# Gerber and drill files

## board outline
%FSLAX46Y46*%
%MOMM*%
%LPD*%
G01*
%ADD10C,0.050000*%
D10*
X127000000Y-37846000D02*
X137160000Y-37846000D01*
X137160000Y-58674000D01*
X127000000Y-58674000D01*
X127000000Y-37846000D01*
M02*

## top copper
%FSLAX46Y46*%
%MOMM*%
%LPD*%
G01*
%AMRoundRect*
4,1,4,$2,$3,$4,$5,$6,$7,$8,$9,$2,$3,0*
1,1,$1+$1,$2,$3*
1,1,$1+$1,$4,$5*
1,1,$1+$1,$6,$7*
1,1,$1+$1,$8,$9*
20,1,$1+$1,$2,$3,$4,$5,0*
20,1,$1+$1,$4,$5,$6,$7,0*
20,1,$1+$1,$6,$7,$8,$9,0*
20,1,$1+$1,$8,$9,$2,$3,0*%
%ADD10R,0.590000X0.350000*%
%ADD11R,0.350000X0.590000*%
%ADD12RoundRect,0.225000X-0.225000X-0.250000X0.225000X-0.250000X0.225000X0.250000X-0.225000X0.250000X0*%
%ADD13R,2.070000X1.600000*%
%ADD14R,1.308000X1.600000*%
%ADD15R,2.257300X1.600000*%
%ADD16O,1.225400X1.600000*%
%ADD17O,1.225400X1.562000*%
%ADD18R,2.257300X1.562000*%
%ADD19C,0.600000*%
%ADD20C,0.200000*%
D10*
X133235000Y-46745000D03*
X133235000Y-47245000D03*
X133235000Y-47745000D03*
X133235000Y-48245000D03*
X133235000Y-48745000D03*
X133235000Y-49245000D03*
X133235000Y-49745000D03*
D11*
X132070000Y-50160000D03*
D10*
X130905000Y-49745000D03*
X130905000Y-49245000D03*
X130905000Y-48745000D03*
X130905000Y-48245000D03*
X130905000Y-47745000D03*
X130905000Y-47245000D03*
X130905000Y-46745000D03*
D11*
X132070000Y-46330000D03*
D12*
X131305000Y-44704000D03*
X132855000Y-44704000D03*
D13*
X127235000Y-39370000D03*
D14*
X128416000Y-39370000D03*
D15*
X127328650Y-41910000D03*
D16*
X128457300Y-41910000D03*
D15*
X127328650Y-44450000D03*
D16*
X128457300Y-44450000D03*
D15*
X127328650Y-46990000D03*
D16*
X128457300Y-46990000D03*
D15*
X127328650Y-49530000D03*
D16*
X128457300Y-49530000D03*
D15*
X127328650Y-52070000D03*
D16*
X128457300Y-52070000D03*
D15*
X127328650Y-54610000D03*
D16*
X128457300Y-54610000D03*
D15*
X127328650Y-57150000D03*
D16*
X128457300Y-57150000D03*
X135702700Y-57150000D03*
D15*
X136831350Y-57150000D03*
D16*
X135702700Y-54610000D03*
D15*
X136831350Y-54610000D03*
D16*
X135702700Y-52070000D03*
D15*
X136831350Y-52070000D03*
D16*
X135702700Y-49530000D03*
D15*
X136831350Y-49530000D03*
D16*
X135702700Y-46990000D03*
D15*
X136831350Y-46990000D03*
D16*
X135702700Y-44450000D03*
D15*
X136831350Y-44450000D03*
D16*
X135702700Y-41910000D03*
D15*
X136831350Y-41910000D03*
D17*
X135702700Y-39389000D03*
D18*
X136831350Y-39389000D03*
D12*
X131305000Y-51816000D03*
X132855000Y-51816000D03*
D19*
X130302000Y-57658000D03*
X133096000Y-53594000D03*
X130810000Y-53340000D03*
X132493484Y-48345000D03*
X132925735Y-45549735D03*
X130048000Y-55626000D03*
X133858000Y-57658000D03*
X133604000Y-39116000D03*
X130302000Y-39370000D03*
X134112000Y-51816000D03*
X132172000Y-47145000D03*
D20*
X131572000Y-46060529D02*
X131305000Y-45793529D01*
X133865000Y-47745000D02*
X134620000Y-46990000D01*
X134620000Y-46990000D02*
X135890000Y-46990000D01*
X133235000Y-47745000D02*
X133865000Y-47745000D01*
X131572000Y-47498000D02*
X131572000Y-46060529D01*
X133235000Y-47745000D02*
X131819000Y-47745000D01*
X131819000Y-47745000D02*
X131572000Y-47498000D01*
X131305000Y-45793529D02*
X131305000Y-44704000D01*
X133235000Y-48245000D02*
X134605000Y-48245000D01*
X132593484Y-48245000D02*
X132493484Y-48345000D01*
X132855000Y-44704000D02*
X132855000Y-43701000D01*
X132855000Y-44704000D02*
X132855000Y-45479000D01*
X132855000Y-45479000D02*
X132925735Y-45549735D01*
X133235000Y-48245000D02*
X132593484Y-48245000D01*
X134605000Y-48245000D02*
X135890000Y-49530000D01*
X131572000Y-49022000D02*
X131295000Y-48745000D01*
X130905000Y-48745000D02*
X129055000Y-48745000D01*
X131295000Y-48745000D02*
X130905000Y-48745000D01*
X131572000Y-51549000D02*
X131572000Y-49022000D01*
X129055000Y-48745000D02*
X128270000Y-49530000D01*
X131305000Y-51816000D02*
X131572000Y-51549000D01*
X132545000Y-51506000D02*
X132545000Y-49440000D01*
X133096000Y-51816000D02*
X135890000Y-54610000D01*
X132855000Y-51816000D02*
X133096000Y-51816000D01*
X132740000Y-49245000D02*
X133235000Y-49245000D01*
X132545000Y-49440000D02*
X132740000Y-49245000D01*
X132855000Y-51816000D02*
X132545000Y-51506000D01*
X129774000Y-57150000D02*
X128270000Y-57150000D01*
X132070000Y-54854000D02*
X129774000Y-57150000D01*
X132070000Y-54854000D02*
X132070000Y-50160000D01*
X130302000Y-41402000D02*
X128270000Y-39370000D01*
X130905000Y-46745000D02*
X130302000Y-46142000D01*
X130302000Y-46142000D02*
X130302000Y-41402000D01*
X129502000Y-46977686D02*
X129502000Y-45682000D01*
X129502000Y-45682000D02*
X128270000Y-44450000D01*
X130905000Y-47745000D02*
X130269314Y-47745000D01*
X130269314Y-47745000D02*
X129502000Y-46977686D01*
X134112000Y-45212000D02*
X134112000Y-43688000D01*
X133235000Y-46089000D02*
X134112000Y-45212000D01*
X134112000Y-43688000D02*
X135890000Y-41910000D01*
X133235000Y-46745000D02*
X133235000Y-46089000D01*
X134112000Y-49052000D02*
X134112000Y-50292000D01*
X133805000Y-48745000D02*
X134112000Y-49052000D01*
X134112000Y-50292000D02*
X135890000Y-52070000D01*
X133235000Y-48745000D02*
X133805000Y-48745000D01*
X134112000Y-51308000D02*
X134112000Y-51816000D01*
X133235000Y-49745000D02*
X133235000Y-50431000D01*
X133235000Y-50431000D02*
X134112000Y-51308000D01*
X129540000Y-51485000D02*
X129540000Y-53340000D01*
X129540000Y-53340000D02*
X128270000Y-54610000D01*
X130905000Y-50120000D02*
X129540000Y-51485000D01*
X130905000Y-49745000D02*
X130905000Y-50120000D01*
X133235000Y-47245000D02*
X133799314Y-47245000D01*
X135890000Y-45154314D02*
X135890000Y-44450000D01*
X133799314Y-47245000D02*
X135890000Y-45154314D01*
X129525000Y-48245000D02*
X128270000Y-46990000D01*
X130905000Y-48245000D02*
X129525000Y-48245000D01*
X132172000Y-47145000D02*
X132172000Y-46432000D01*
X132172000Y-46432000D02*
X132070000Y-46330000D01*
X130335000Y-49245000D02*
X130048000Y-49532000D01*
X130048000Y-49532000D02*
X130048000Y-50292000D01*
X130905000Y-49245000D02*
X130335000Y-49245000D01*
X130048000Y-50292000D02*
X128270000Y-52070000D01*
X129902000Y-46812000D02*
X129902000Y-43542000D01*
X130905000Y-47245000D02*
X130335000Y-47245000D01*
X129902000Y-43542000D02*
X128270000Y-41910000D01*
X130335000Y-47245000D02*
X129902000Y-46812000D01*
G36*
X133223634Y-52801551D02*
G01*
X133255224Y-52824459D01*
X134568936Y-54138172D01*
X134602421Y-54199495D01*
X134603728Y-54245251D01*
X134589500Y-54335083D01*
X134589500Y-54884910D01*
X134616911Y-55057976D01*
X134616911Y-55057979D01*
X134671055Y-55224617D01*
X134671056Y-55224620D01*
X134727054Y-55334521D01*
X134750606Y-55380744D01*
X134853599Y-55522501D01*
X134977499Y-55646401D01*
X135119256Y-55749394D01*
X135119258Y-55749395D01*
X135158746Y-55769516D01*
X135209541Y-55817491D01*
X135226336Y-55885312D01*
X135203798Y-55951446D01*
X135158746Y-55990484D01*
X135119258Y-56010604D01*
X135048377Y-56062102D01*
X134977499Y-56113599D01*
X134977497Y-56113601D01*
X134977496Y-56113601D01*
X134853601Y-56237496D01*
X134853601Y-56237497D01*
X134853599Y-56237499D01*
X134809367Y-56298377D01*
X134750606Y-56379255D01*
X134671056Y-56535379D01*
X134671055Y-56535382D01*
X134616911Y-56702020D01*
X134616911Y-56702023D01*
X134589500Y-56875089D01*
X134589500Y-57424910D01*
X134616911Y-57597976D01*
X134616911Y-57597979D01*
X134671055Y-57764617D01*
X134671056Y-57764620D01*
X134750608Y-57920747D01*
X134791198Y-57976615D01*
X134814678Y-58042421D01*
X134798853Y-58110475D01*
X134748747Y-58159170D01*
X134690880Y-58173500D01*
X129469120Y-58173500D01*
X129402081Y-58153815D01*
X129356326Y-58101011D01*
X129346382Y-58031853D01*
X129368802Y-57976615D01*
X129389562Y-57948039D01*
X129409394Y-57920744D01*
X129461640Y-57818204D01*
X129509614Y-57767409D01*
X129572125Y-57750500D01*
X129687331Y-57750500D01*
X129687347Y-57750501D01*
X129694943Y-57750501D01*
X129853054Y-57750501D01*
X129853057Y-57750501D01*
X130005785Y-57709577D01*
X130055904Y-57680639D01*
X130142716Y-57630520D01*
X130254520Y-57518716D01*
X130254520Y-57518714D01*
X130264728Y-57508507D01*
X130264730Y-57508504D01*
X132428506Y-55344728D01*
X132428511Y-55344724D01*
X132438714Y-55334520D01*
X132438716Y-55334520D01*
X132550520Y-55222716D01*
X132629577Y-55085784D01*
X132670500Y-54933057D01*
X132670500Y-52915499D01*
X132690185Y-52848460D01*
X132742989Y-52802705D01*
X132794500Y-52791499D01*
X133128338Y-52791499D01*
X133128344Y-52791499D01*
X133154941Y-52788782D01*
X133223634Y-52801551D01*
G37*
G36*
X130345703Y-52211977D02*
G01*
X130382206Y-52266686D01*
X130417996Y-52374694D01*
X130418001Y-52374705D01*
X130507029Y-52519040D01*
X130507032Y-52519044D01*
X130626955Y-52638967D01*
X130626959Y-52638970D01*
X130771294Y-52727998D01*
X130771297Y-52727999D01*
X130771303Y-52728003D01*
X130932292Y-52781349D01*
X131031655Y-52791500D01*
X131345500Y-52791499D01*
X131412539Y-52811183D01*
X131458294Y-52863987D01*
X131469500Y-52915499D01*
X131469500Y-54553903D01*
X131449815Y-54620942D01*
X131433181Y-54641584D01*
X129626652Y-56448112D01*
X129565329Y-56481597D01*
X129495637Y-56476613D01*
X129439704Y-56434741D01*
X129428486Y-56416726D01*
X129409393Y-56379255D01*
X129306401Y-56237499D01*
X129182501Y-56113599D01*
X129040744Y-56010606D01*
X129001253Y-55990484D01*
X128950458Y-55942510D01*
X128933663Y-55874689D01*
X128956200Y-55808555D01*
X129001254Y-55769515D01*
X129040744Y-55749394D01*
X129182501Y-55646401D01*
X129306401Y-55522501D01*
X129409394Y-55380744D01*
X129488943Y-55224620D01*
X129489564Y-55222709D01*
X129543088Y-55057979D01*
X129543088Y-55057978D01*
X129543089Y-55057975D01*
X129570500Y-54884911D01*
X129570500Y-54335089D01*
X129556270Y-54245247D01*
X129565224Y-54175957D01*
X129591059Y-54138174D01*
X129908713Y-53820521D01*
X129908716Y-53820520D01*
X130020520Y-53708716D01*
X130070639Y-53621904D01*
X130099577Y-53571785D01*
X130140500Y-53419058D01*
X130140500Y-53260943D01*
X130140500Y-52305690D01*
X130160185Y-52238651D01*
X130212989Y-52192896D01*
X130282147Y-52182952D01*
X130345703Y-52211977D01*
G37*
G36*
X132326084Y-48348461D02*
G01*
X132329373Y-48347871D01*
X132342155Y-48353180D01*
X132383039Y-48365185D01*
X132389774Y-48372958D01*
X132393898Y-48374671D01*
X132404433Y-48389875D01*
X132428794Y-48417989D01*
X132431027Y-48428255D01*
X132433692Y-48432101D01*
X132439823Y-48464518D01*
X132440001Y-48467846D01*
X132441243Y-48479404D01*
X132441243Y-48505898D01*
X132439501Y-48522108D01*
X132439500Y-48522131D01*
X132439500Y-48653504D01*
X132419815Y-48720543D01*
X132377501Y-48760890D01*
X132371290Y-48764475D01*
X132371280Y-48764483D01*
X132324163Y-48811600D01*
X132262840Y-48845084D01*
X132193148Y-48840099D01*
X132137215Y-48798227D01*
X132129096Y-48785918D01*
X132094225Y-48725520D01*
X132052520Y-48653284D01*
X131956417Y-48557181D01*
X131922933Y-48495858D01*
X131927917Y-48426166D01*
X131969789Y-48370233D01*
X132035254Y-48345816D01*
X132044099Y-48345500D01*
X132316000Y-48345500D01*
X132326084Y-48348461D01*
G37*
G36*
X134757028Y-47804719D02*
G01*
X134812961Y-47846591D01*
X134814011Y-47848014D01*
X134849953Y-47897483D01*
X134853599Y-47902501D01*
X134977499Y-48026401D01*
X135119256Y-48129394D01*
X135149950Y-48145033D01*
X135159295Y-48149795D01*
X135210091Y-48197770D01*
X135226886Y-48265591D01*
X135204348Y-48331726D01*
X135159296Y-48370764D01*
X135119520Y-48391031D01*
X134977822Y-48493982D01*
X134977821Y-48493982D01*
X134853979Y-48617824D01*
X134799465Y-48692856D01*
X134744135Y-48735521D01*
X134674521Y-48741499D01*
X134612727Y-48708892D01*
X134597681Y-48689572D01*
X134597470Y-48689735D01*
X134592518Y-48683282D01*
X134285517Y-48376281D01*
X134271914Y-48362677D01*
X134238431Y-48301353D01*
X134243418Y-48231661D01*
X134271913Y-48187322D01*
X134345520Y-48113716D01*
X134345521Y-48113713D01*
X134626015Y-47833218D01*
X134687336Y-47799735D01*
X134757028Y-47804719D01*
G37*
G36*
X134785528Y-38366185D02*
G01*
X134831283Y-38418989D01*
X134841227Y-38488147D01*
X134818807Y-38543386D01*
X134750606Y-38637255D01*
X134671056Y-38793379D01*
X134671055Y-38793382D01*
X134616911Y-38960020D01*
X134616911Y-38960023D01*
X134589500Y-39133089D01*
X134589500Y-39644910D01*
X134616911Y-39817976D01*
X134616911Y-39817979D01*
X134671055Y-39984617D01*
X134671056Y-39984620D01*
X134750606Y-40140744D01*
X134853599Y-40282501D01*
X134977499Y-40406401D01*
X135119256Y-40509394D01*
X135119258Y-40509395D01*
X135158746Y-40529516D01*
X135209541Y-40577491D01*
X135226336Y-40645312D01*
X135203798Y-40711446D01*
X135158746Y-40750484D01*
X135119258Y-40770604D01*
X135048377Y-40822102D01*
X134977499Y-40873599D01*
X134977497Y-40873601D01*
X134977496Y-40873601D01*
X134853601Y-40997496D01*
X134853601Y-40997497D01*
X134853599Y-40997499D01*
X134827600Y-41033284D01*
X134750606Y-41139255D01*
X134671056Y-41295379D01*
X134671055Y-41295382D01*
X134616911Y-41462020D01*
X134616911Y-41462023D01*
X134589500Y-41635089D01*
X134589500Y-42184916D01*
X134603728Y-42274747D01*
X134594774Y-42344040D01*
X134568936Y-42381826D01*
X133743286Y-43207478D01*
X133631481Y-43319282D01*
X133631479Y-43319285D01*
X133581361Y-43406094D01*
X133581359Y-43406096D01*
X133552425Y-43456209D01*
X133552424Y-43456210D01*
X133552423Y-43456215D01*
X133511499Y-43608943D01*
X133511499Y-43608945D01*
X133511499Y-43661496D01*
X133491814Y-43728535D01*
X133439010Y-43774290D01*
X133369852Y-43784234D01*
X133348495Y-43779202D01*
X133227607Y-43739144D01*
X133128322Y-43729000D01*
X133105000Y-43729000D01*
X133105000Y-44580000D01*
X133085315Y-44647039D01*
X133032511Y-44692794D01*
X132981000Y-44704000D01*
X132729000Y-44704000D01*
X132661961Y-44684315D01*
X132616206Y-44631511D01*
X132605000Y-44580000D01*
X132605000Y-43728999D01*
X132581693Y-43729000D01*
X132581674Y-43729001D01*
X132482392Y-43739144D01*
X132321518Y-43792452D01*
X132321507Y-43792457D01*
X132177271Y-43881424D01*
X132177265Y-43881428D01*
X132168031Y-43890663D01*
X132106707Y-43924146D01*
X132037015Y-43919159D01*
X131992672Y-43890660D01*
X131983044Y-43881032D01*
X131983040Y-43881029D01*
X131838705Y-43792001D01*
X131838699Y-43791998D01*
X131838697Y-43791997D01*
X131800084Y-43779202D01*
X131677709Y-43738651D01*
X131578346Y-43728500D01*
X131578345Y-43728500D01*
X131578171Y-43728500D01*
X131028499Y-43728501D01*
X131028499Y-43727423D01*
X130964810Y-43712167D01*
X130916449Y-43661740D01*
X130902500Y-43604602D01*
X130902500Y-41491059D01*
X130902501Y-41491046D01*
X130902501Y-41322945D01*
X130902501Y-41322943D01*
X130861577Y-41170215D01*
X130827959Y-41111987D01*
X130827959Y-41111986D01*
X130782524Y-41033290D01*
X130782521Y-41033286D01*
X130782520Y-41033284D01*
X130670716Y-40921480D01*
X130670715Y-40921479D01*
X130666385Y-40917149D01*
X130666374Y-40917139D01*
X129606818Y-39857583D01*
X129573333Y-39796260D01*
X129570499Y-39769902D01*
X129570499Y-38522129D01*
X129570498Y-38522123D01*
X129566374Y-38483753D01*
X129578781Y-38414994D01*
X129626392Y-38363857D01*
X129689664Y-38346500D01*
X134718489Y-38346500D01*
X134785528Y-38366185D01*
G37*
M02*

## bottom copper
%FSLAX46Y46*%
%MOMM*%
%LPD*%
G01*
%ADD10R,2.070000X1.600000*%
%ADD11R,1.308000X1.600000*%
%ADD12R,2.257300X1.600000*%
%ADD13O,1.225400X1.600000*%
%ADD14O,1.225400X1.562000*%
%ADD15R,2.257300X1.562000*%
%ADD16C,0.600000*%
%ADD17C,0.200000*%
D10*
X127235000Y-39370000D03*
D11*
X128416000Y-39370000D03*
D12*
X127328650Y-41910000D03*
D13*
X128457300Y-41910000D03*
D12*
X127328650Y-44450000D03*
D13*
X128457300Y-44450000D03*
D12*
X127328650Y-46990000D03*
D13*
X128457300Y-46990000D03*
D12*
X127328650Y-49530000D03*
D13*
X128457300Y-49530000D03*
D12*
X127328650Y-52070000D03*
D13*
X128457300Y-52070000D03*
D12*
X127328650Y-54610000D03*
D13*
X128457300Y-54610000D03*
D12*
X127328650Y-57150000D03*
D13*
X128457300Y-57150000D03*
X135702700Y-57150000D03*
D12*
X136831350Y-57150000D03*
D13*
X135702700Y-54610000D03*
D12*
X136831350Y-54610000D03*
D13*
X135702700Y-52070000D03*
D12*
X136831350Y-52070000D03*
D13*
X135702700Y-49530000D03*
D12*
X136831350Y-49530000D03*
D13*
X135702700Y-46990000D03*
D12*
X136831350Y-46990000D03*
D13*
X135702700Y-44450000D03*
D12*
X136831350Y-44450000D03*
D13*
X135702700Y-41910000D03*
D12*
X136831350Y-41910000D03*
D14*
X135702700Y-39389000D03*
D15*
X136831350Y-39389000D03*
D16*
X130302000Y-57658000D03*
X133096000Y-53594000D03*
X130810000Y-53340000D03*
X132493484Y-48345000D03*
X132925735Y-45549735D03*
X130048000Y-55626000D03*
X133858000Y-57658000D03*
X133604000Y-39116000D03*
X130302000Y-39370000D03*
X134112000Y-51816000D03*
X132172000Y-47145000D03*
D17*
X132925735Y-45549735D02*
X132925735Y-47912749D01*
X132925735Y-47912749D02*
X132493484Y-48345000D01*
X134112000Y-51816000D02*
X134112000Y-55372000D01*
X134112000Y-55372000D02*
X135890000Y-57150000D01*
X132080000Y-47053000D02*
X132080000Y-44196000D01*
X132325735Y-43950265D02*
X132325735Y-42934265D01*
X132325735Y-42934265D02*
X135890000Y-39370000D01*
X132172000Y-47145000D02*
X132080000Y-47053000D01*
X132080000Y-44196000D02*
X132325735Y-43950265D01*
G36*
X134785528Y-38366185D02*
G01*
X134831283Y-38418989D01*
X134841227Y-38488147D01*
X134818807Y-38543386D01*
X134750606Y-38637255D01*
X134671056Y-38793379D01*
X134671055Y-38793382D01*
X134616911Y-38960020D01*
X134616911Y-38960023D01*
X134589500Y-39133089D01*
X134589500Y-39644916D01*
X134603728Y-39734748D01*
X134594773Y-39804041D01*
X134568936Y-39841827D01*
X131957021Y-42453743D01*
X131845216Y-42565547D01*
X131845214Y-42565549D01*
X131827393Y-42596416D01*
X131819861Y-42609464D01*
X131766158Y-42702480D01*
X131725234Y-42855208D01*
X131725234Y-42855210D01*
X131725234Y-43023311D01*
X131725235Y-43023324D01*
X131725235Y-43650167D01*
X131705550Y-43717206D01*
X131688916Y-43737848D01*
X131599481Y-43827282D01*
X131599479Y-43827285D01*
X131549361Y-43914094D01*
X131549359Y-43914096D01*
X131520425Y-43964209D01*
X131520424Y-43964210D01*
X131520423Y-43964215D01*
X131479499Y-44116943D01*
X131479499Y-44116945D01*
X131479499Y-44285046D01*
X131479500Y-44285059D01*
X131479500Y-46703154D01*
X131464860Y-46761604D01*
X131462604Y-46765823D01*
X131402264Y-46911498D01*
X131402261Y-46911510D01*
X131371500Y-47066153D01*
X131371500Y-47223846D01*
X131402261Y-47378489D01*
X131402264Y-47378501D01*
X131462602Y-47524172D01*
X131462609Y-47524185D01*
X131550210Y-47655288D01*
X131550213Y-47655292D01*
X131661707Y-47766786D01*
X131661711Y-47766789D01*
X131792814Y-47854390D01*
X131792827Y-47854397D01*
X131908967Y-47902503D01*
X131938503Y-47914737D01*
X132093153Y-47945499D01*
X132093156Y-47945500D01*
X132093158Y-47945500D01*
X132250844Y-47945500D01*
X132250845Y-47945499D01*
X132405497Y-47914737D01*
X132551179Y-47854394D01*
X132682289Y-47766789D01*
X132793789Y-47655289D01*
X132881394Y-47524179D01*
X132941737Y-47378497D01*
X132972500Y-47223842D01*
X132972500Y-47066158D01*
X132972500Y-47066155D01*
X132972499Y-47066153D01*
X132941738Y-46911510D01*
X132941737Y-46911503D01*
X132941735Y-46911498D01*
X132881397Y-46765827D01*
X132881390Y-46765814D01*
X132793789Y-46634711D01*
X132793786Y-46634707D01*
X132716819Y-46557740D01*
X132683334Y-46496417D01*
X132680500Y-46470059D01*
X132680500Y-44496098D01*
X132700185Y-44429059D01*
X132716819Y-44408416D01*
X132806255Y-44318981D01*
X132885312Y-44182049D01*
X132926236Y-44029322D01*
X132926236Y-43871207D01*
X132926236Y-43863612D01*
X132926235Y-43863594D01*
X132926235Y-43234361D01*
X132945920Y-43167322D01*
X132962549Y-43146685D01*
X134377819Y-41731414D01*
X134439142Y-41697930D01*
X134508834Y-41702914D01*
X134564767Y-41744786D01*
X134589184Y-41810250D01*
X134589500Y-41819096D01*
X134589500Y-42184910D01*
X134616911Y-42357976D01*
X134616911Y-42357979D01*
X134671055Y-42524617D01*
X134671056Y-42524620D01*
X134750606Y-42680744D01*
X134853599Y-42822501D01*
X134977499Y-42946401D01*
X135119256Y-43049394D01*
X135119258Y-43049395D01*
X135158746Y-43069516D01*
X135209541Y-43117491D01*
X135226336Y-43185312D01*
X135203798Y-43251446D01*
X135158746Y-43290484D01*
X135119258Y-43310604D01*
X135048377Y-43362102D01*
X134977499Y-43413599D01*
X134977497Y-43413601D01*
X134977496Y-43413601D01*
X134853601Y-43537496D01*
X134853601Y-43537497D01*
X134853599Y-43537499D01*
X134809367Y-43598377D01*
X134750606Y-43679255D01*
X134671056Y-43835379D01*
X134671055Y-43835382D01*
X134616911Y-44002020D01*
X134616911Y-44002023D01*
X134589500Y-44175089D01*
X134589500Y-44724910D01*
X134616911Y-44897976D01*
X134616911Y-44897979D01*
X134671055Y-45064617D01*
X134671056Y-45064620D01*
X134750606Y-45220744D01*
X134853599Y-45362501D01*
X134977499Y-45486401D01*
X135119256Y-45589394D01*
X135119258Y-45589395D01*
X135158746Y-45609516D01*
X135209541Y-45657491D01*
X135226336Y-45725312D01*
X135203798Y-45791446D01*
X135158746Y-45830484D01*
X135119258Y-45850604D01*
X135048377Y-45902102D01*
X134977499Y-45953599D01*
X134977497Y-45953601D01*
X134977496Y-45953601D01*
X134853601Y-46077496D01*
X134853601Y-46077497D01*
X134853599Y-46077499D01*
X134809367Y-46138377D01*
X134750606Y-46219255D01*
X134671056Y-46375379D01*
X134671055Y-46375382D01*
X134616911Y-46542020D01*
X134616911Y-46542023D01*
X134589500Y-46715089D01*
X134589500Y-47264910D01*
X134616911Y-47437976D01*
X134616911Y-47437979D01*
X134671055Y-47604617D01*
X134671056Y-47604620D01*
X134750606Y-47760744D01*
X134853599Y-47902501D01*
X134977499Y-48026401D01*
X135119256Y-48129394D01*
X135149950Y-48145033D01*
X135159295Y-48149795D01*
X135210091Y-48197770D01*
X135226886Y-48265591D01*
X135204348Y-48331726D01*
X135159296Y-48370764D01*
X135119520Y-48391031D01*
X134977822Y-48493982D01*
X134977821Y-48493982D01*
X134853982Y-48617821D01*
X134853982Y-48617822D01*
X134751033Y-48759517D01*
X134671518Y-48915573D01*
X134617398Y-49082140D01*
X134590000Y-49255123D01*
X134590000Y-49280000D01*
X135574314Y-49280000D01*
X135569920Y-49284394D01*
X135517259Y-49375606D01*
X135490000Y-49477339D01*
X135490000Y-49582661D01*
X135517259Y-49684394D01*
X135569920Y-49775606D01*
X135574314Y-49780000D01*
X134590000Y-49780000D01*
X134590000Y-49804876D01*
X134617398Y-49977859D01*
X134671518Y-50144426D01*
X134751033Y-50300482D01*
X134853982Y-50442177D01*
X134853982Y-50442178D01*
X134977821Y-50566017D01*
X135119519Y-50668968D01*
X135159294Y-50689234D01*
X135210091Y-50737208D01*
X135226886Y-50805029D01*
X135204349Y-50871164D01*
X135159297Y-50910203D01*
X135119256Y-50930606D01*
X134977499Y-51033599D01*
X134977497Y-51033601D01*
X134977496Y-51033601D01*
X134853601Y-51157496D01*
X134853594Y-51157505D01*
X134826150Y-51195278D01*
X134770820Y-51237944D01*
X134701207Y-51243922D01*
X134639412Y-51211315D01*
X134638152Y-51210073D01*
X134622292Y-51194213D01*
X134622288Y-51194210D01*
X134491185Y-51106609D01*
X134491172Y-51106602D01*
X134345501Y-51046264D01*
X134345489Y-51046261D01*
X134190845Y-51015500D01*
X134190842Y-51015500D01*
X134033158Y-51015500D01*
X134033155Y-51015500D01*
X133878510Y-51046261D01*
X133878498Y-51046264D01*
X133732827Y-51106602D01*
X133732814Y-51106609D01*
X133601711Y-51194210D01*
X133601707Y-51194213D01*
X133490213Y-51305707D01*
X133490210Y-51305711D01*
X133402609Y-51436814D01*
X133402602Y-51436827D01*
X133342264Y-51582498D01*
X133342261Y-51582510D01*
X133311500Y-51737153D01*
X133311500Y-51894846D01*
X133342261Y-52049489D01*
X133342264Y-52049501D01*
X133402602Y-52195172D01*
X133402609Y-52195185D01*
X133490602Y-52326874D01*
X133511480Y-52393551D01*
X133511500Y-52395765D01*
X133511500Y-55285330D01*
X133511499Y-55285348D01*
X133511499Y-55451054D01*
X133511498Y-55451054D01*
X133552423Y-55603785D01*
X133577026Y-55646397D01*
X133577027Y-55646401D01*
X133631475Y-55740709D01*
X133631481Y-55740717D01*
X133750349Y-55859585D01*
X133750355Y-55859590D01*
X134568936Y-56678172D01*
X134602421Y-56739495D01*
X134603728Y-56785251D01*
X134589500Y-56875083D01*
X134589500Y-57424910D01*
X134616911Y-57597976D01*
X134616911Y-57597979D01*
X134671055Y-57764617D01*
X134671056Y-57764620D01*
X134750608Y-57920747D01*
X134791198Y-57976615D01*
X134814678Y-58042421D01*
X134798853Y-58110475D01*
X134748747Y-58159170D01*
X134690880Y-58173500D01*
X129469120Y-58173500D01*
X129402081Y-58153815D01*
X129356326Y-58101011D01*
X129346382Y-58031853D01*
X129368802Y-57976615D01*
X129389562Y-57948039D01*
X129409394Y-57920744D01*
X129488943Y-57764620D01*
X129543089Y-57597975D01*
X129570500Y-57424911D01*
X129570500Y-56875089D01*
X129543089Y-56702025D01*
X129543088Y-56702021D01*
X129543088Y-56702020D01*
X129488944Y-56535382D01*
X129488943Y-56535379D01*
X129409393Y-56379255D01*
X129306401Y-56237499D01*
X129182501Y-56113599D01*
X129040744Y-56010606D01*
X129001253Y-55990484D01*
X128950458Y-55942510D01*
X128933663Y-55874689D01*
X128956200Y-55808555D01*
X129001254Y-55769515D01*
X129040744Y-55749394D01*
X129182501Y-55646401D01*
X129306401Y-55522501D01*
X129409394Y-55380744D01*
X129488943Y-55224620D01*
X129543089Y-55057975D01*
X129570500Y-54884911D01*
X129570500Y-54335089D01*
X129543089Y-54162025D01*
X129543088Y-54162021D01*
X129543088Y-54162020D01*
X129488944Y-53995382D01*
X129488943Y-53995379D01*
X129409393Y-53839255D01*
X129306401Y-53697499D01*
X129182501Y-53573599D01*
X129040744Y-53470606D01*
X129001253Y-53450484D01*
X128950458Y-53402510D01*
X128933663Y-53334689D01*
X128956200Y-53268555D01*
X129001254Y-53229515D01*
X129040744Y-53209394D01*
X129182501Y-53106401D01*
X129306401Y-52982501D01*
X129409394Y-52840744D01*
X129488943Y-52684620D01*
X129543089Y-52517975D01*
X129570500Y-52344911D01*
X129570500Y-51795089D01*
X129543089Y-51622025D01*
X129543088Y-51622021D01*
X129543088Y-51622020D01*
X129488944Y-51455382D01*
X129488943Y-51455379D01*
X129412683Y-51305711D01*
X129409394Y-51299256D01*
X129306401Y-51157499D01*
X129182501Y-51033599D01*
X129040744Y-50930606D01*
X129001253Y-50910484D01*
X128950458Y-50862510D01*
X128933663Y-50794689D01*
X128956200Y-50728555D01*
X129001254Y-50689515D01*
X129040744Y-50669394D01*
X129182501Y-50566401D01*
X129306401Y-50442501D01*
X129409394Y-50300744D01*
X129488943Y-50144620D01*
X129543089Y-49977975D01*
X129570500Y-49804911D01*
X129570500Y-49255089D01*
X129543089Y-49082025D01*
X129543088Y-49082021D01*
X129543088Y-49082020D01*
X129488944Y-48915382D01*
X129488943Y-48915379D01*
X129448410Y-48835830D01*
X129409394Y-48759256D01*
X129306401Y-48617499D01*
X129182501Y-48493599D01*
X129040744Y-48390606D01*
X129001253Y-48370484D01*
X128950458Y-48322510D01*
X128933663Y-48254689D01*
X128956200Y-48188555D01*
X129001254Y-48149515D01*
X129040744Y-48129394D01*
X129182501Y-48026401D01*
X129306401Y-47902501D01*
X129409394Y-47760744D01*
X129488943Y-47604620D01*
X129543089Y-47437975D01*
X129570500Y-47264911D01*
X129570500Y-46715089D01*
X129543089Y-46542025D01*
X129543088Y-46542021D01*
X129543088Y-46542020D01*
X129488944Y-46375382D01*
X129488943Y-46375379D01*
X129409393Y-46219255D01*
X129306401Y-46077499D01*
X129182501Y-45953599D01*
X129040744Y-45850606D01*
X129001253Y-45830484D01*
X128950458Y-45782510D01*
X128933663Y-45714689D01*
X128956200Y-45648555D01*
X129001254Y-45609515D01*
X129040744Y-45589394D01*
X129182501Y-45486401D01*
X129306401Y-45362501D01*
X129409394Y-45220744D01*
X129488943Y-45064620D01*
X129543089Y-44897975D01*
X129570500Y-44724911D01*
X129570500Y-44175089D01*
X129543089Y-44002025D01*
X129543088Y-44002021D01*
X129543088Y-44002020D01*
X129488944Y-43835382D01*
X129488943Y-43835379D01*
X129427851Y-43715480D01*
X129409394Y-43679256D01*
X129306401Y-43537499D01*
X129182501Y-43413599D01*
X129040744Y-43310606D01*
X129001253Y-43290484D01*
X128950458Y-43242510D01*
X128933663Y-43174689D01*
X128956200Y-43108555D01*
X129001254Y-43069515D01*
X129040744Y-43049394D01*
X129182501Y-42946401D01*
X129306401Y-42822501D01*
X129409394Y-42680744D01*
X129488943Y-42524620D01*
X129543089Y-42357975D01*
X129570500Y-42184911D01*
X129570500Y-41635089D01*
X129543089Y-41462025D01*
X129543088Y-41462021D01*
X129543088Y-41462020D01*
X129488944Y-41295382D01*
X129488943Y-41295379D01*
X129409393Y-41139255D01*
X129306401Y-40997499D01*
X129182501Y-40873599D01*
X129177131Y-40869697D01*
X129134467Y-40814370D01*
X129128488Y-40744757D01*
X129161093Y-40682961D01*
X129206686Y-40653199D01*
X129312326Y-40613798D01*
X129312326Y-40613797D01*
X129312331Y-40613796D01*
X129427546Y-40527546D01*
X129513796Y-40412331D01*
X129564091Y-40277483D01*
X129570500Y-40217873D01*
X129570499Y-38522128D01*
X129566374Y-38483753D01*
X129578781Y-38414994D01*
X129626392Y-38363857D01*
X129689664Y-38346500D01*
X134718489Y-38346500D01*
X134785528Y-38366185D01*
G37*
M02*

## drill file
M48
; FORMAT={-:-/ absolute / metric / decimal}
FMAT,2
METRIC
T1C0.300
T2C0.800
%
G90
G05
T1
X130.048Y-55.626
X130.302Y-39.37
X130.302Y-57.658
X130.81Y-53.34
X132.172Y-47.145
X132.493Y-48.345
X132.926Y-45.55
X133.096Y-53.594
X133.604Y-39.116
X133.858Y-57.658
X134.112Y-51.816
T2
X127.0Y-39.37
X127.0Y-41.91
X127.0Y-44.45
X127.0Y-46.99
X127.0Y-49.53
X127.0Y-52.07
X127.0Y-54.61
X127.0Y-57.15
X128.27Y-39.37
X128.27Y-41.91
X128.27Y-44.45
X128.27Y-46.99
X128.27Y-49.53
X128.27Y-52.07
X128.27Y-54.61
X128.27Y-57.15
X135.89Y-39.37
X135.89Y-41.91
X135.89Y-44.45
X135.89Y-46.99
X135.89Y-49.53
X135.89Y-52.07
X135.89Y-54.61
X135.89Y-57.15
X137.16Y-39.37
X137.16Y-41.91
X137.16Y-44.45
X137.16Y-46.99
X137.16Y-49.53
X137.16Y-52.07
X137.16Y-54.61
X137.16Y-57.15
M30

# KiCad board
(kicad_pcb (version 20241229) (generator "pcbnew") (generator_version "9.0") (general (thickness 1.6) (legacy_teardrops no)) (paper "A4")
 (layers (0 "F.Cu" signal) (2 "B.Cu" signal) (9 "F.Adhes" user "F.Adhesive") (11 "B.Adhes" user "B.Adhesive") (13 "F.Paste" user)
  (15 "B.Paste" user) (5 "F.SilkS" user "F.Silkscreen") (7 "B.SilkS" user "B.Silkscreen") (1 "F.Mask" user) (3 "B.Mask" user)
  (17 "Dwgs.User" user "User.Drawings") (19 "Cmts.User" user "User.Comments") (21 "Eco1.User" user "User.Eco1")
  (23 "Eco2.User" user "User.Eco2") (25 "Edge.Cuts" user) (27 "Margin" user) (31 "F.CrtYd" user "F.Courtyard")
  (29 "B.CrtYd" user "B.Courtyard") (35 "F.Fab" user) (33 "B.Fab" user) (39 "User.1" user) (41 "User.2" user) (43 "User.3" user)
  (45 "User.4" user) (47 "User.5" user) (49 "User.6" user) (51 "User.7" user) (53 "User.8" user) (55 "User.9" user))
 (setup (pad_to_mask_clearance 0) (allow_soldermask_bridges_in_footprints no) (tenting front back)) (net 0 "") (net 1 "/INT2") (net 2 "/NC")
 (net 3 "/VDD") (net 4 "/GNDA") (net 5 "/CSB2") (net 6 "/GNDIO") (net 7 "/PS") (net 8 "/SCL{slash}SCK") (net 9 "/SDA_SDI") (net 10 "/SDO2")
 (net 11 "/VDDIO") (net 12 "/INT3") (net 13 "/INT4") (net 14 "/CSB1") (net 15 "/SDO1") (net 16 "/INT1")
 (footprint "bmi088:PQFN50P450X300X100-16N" (layer "F.Cu") (at 132.07 48.245 -90)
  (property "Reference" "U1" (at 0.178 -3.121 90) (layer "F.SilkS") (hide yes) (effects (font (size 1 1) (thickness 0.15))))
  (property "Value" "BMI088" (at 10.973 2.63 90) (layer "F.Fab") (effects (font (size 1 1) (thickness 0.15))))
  (pad "1" smd rect (at -1.5 -1.165 270) (size 0.35 0.59) (layers "F.Cu" "F.Mask" "F.Paste") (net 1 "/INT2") (solder_mask_margin 0.03))
  (pad "2" smd rect (at -1 -1.165 270) (size 0.35 0.59) (layers "F.Cu" "F.Mask" "F.Paste") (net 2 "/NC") (solder_mask_margin 0.03))
  (pad "3" smd rect (at -0.5 -1.165 270) (size 0.35 0.59) (layers "F.Cu" "F.Mask" "F.Paste") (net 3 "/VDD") (solder_mask_margin 0.03))
  (pad "4" smd rect (at 0 -1.165 270) (size 0.35 0.59) (layers "F.Cu" "F.Mask" "F.Paste") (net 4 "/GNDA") (solder_mask_margin 0.03))
  (pad "5" smd rect (at 0.5 -1.165 270) (size 0.35 0.59) (layers "F.Cu" "F.Mask" "F.Paste") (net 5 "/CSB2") (solder_mask_margin 0.03))
  (pad "6" smd rect (at 1 -1.165 270) (size 0.35 0.59) (layers "F.Cu" "F.Mask" "F.Paste") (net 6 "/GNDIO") (solder_mask_margin 0.03))
  (pad "7" smd rect (at 1.5 -1.165 270) (size 0.35 0.59) (layers "F.Cu" "F.Mask" "F.Paste") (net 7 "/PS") (solder_mask_margin 0.03))
  (pad "8" smd rect (at 1.915 0 270) (size 0.59 0.35) (layers "F.Cu" "F.Mask" "F.Paste") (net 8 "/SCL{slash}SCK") (solder_mask_margin 0.03))
  (pad "9" smd rect (at 1.5 1.165 270) (size 0.35 0.59) (layers "F.Cu" "F.Mask" "F.Paste") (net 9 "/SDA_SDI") (solder_mask_margin 0.03))
  (pad "10" smd rect (at 1 1.165 270) (size 0.35 0.59) (layers "F.Cu" "F.Mask" "F.Paste") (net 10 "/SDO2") (solder_mask_margin 0.03))
  (pad "11" smd rect (at 0.5 1.165 270) (size 0.35 0.59) (layers "F.Cu" "F.Mask" "F.Paste") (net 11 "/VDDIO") (solder_mask_margin 0.03))
  (pad "12" smd rect (at 0 1.165 270) (size 0.35 0.59) (layers "F.Cu" "F.Mask" "F.Paste") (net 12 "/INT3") (solder_mask_margin 0.03))
  (pad "13" smd rect (at -0.5 1.165 270) (size 0.35 0.59) (layers "F.Cu" "F.Mask" "F.Paste") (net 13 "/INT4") (solder_mask_margin 0.03))
  (pad "14" smd rect (at -1 1.165 270) (size 0.35 0.59) (layers "F.Cu" "F.Mask" "F.Paste") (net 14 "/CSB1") (solder_mask_margin 0.03))
  (pad "15" smd rect (at -1.5 1.165 270) (size 0.35 0.59) (layers "F.Cu" "F.Mask" "F.Paste") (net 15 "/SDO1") (solder_mask_margin 0.03))
  (pad "16" smd rect (at -1.915 0 270) (size 0.59 0.35) (layers "F.Cu" "F.Mask" "F.Paste") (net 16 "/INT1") (solder_mask_margin 0.03)))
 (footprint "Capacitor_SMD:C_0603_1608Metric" (layer "F.Cu") (at 132.08 44.704)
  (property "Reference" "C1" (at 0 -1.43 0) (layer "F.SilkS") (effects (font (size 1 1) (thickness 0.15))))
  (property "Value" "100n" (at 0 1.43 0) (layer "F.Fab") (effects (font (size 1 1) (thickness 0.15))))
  (pad "1" smd roundrect (at -0.775 0) (size 0.9 0.95) (layers "F.Cu" "F.Mask" "F.Paste") (roundrect_rratio 0.25) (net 3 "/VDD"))
  (pad "2" smd roundrect (at 0.775 0) (size 0.9 0.95) (layers "F.Cu" "F.Mask" "F.Paste") (roundrect_rratio 0.25) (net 4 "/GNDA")))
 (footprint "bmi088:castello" (layer "F.Cu") (at 128.27 39.37)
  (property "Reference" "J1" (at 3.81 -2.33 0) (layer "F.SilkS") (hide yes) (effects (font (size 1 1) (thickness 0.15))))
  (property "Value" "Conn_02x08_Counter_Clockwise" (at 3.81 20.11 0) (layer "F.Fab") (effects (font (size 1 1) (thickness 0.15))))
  (pad "1" thru_hole rect (at -1.27 0) (size 2.07 1.6) (drill 0.8 (offset 0.235 0)) (layers "*.Cu" "*.Mask") (remove_unused_layers no)
   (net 15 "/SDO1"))
  (pad "1" thru_hole rect (at 0 0) (size 1.308 1.6) (drill 0.8 (offset 0.146 0)) (layers "*.Cu" "*.Mask") (remove_unused_layers no)
   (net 15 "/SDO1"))
  (pad "2" thru_hole rect (at -1.27 2.54) (size 2.2573 1.6) (drill 0.8 (offset 0.32865 0)) (layers "*.Cu" "*.Mask")
   (remove_unused_layers no) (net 14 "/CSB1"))
  (pad "2" thru_hole oval (at 0 2.54) (size 1.2254 1.6) (drill 0.8 (offset 0.1873 0)) (layers "*.Cu" "*.Mask") (remove_unused_layers no)
   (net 14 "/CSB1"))
  (pad "3" thru_hole rect (at -1.27 5.08) (size 2.2573 1.6) (drill 0.8 (offset 0.32865 0)) (layers "*.Cu" "*.Mask")
   (remove_unused_layers no) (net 13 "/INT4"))
  (pad "3" thru_hole oval (at 0 5.08) (size 1.2254 1.6) (drill 0.8 (offset 0.1873 0)) (layers "*.Cu" "*.Mask") (remove_unused_layers no)
   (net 13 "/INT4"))
  (pad "4" thru_hole rect (at -1.27 7.62) (size 2.2573 1.6) (drill 0.8 (offset 0.32865 0)) (layers "*.Cu" "*.Mask")
   (remove_unused_layers no) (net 12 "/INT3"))
  (pad "4" thru_hole oval (at 0 7.62) (size 1.2254 1.6) (drill 0.8 (offset 0.1873 0)) (layers "*.Cu" "*.Mask") (remove_unused_layers no)
   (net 12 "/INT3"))
  (pad "5" thru_hole rect (at -1.27 10.16) (size 2.2573 1.6) (drill 0.8 (offset 0.32865 0)) (layers "*.Cu" "*.Mask")
   (remove_unused_layers no) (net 11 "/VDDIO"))
  (pad "5" thru_hole oval (at 0 10.16) (size 1.2254 1.6) (drill 0.8 (offset 0.1873 0)) (layers "*.Cu" "*.Mask") (remove_unused_layers no)
   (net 11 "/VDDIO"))
  (pad "6" thru_hole rect (at -1.27 12.7 180) (size 2.2573 1.6) (drill 0.8 (offset -0.32865 0)) (layers "*.Cu" "*.Mask")
   (remove_unused_layers no) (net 10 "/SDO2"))
  (pad "6" thru_hole oval (at 0 12.7) (size 1.2254 1.6) (drill 0.8 (offset 0.1873 0)) (layers "*.Cu" "*.Mask") (remove_unused_layers no)
   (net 10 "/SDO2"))
  (pad "7" thru_hole rect (at -1.27 15.24) (size 2.2573 1.6) (drill 0.8 (offset 0.32865 0)) (layers "*.Cu" "*.Mask")
   (remove_unused_layers no) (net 9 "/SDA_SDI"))
  (pad "7" thru_hole oval (at 0 15.24) (size 1.2254 1.6) (drill 0.8 (offset 0.1873 0)) (layers "*.Cu" "*.Mask") (remove_unused_layers no)
   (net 9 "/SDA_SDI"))
  (pad "8" thru_hole rect (at -1.27 17.78) (size 2.2573 1.6) (drill 0.8 (offset 0.32865 0)) (layers "*.Cu" "*.Mask")
   (remove_unused_layers no) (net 8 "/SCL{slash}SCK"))
  (pad "8" thru_hole oval (at 0 17.78) (size 1.2254 1.6) (drill 0.8 (offset 0.1873 0)) (layers "*.Cu" "*.Mask") (remove_unused_layers no)
   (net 8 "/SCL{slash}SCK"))
  (pad "9" thru_hole oval (at 7.62 17.78) (size 1.2254 1.6) (drill 0.8 (offset -0.1873 0)) (layers "*.Cu" "*.Mask")
   (remove_unused_layers no) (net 7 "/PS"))
  (pad "9" thru_hole rect (at 8.89 17.78) (size 2.2573 1.6) (drill 0.8 (offset -0.32865 0)) (layers "*.Cu" "*.Mask")
   (remove_unused_layers no) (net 7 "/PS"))
  (pad "10" thru_hole oval (at 7.62 15.24) (size 1.2254 1.6) (drill 0.8 (offset -0.1873 0)) (layers "*.Cu" "*.Mask")
   (remove_unused_layers no) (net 6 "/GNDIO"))
  (pad "10" thru_hole rect (at 8.89 15.24) (size 2.2573 1.6) (drill 0.8 (offset -0.32865 0)) (layers "*.Cu" "*.Mask")
   (remove_unused_layers no) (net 6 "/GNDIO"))
  (pad "11" thru_hole oval (at 7.62 12.7) (size 1.2254 1.6) (drill 0.8 (offset -0.1873 0)) (layers "*.Cu" "*.Mask")
   (remove_unused_layers no) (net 5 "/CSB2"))
  (pad "11" thru_hole rect (at 8.89 12.7) (size 2.2573 1.6) (drill 0.8 (offset -0.32865 0)) (layers "*.Cu" "*.Mask")
   (remove_unused_layers no) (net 5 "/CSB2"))
  (pad "12" thru_hole oval (at 7.62 10.16) (size 1.2254 1.6) (drill 0.8 (offset -0.1873 0)) (layers "*.Cu" "*.Mask")
   (remove_unused_layers no) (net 4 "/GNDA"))
  (pad "12" thru_hole rect (at 8.89 10.16) (size 2.2573 1.6) (drill 0.8 (offset -0.32865 0)) (layers "*.Cu" "*.Mask")
   (remove_unused_layers no) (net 4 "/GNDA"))
  (pad "13" thru_hole oval (at 7.62 7.62) (size 1.2254 1.6) (drill 0.8 (offset -0.1873 0)) (layers "*.Cu" "*.Mask")
   (remove_unused_layers no) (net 3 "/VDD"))
  (pad "13" thru_hole rect (at 8.89 7.62) (size 2.2573 1.6) (drill 0.8 (offset -0.32865 0)) (layers "*.Cu" "*.Mask")
   (remove_unused_layers no) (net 3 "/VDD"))
  (pad "14" thru_hole oval (at 7.62 5.08) (size 1.2254 1.6) (drill 0.8 (offset -0.1873 0)) (layers "*.Cu" "*.Mask")
   (remove_unused_layers no) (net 2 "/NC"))
  (pad "14" thru_hole rect (at 8.89 5.08) (size 2.2573 1.6) (drill 0.8 (offset -0.32865 0)) (layers "*.Cu" "*.Mask")
   (remove_unused_layers no) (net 2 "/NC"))
  (pad "15" thru_hole oval (at 7.62 2.54) (size 1.2254 1.6) (drill 0.8 (offset -0.1873 0)) (layers "*.Cu" "*.Mask")
   (remove_unused_layers no) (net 1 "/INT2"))
  (pad "15" thru_hole rect (at 8.89 2.54) (size 2.2573 1.6) (drill 0.8 (offset -0.32865 0)) (layers "*.Cu" "*.Mask")
   (remove_unused_layers no) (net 1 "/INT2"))
  (pad "16" thru_hole oval (at 7.62 0) (size 1.2254 1.562) (drill 0.8 (offset -0.1873 0.019)) (layers "*.Cu" "*.Mask")
   (remove_unused_layers no) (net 16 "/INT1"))
  (pad "16" thru_hole rect (at 8.89 0) (size 2.2573 1.562) (drill 0.8 (offset -0.32865 0.019)) (layers "*.Cu" "*.Mask")
   (remove_unused_layers no) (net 16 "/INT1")))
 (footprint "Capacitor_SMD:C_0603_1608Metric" (layer "F.Cu") (at 132.08 51.816)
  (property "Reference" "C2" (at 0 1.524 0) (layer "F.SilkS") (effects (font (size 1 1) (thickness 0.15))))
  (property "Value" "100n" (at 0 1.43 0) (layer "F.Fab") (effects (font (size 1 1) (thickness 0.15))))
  (pad "1" smd roundrect (at -0.775 0) (size 0.9 0.95) (layers "F.Cu" "F.Mask" "F.Paste") (roundrect_rratio 0.25) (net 11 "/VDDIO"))
  (pad "2" smd roundrect (at 0.775 0) (size 0.9 0.95) (layers "F.Cu" "F.Mask" "F.Paste") (roundrect_rratio 0.25) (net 6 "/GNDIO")))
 (gr_rect (start 127 37.846) (end 137.16 58.674) (stroke (width 0.05) (type default)) (fill no) (layer "Edge.Cuts"))
 (segment (start 131.572 46.060529) (end 131.305 45.793529) (width 0.2) (layer "F.Cu") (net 3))
 (segment (start 133.865 47.745) (end 134.62 46.99) (width 0.2) (layer "F.Cu") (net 3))
 (segment (start 134.62 46.99) (end 135.89 46.99) (width 0.2) (layer "F.Cu") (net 3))
 (segment (start 133.235 47.745) (end 133.865 47.745) (width 0.2) (layer "F.Cu") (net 3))
 (segment (start 131.572 47.498) (end 131.572 46.060529) (width 0.2) (layer "F.Cu") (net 3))
 (segment (start 133.235 47.745) (end 131.819 47.745) (width 0.2) (layer "F.Cu") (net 3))
 (segment (start 131.819 47.745) (end 131.572 47.498) (width 0.2) (layer "F.Cu") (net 3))
 (segment (start 131.305 45.793529) (end 131.305 44.704) (width 0.2) (layer "F.Cu") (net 3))
 (segment (start 133.235 48.245) (end 134.605 48.245) (width 0.2) (layer "F.Cu") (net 4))
 (segment (start 132.593484 48.245) (end 132.493484 48.345) (width 0.2) (layer "F.Cu") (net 4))
 (segment (start 132.855 44.704) (end 132.855 43.701) (width 0.2) (layer "F.Cu") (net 4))
 (segment (start 132.855 44.704) (end 132.855 45.479) (width 0.2) (layer "F.Cu") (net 4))
 (segment (start 132.855 45.479) (end 132.925735 45.549735) (width 0.2) (layer "F.Cu") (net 4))
 (segment (start 133.235 48.245) (end 132.593484 48.245) (width 0.2) (layer "F.Cu") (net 4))
 (segment (start 134.605 48.245) (end 135.89 49.53) (width 0.2) (layer "F.Cu") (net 4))
 (via (at 130.302 57.658) (size 0.6) (drill 0.3) (layers "F.Cu" "B.Cu") (free yes) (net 4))
 (via (at 133.096 53.594) (size 0.6) (drill 0.3) (layers "F.Cu" "B.Cu") (free yes) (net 4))
 (via (at 130.81 53.34) (size 0.6) (drill 0.3) (layers "F.Cu" "B.Cu") (free yes) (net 4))
 (via (at 132.493484 48.345) (size 0.6) (drill 0.3) (layers "F.Cu" "B.Cu") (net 4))
 (via (at 132.925735 45.549735) (size 0.6) (drill 0.3) (layers "F.Cu" "B.Cu") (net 4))
 (via (at 130.048 55.626) (size 0.6) (drill 0.3) (layers "F.Cu" "B.Cu") (free yes) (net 4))
 (via (at 133.858 57.658) (size 0.6) (drill 0.3) (layers "F.Cu" "B.Cu") (free yes) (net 4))
 (via (at 133.604 39.116) (size 0.6) (drill 0.3) (layers "F.Cu" "B.Cu") (free yes) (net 4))
 (via (at 130.302 39.37) (size 0.6) (drill 0.3) (layers "F.Cu" "B.Cu") (free yes) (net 4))
 (segment (start 132.925735 45.549735) (end 132.925735 47.912749) (width 0.2) (layer "B.Cu") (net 4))
 (segment (start 132.925735 47.912749) (end 132.493484 48.345) (width 0.2) (layer "B.Cu") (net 4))
 (segment (start 131.572 49.022) (end 131.295 48.745) (width 0.2) (layer "F.Cu") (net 11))
 (segment (start 130.905 48.745) (end 129.055 48.745) (width 0.2) (layer "F.Cu") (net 11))
 (segment (start 131.295 48.745) (end 130.905 48.745) (width 0.2) (layer "F.Cu") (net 11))
 (segment (start 131.572 51.549) (end 131.572 49.022) (width 0.2) (layer "F.Cu") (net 11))
 (segment (start 129.055 48.745) (end 128.27 49.53) (width 0.2) (layer "F.Cu") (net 11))
 (segment (start 131.305 51.816) (end 131.572 51.549) (width 0.2) (layer "F.Cu") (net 11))
 (segment (start 132.545 51.506) (end 132.545 49.44) (width 0.2) (layer "F.Cu") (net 6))
 (segment (start 133.096 51.816) (end 135.89 54.61) (width 0.2) (layer "F.Cu") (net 6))
 (segment (start 132.855 51.816) (end 133.096 51.816) (width 0.2) (layer "F.Cu") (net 6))
 (segment (start 132.74 49.245) (end 133.235 49.245) (width 0.2) (layer "F.Cu") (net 6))
 (segment (start 132.545 49.44) (end 132.74 49.245) (width 0.2) (layer "F.Cu") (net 6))
 (segment (start 132.855 51.816) (end 132.545 51.506) (width 0.2) (layer "F.Cu") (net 6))
 (segment (start 129.774 57.15) (end 128.27 57.15) (width 0.2) (layer "F.Cu") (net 8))
 (segment (start 132.07 54.854) (end 129.774 57.15) (width 0.2) (layer "F.Cu") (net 8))
 (segment (start 132.07 54.854) (end 132.07 50.16) (width 0.2) (layer "F.Cu") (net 8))
 (segment (start 130.302 41.402) (end 128.27 39.37) (width 0.2) (layer "F.Cu") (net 15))
 (segment (start 130.905 46.745) (end 130.302 46.142) (width 0.2) (layer "F.Cu") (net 15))
 (segment (start 130.302 46.142) (end 130.302 41.402) (width 0.2) (layer "F.Cu") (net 15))
 (segment (start 129.502 46.977686) (end 129.502 45.682) (width 0.2) (layer "F.Cu") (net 13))
 (segment (start 129.502 45.682) (end 128.27 44.45) (width 0.2) (layer "F.Cu") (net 13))
 (segment (start 130.905 47.745) (end 130.269314 47.745) (width 0.2) (layer "F.Cu") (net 13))
 (segment (start 130.269314 47.745) (end 129.502 46.977686) (width 0.2) (layer "F.Cu") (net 13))
 (segment (start 134.112 45.212) (end 134.112 43.688) (width 0.2) (layer "F.Cu") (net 1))
 (segment (start 133.235 46.089) (end 134.112 45.212) (width 0.2) (layer "F.Cu") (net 1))
 (segment (start 134.112 43.688) (end 135.89 41.91) (width 0.2) (layer "F.Cu") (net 1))
 (segment (start 133.235 46.745) (end 133.235 46.089) (width 0.2) (layer "F.Cu") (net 1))
 (segment (start 134.112 49.052) (end 134.112 50.292) (width 0.2) (layer "F.Cu") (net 5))
 (segment (start 133.805 48.745) (end 134.112 49.052) (width 0.2) (layer "F.Cu") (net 5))
 (segment (start 134.112 50.292) (end 135.89 52.07) (width 0.2) (layer "F.Cu") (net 5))
 (segment (start 133.235 48.745) (end 133.805 48.745) (width 0.2) (layer "F.Cu") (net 5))
 (segment (start 134.112 51.308) (end 134.112 51.816) (width 0.2) (layer "F.Cu") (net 7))
 (segment (start 133.235 49.745) (end 133.235 50.431) (width 0.2) (layer "F.Cu") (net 7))
 (segment (start 133.235 50.431) (end 134.112 51.308) (width 0.2) (layer "F.Cu") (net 7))
 (via (at 134.112 51.816) (size 0.6) (drill 0.3) (layers "F.Cu" "B.Cu") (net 7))
 (segment (start 134.112 51.816) (end 134.112 55.372) (width 0.2) (layer "B.Cu") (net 7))
 (segment (start 134.112 55.372) (end 135.89 57.15) (width 0.2) (layer "B.Cu") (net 7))
 (segment (start 129.54 51.485) (end 129.54 53.34) (width 0.2) (layer "F.Cu") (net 9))
 (segment (start 129.54 53.34) (end 128.27 54.61) (width 0.2) (layer "F.Cu") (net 9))
 (segment (start 130.905 50.12) (end 129.54 51.485) (width 0.2) (layer "F.Cu") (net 9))
 (segment (start 130.905 49.745) (end 130.905 50.12) (width 0.2) (layer "F.Cu") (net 9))
 (segment (start 133.235 47.245) (end 133.799314 47.245) (width 0.2) (layer "F.Cu") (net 2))
 (segment (start 135.89 45.154314) (end 135.89 44.45) (width 0.2) (layer "F.Cu") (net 2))
 (segment (start 133.799314 47.245) (end 135.89 45.154314) (width 0.2) (layer "F.Cu") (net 2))
 (segment (start 129.525 48.245) (end 128.27 46.99) (width 0.2) (layer "F.Cu") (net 12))
 (segment (start 130.905 48.245) (end 129.525 48.245) (width 0.2) (layer "F.Cu") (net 12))
 (segment (start 132.172 47.145) (end 132.172 46.432) (width 0.2) (layer "F.Cu") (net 16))
 (segment (start 132.172 46.432) (end 132.07 46.33) (width 0.2) (layer "F.Cu") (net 16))
 (via (at 132.172 47.145) (size 0.6) (drill 0.3) (layers "F.Cu" "B.Cu") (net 16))
 (segment (start 132.08 47.053) (end 132.08 44.196) (width 0.2) (layer "B.Cu") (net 16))
 (segment (start 132.325735 43.950265) (end 132.325735 42.934265) (width 0.2) (layer "B.Cu") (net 16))
 (segment (start 132.325735 42.934265) (end 135.89 39.37) (width 0.2) (layer "B.Cu") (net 16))
 (segment (start 132.172 47.145) (end 132.08 47.053) (width 0.2) (layer "B.Cu") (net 16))
 (segment (start 132.08 44.196) (end 132.325735 43.950265) (width 0.2) (layer "B.Cu") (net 16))
 (segment (start 130.335 49.245) (end 130.048 49.532) (width 0.2) (layer "F.Cu") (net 10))
 (segment (start 130.048 49.532) (end 130.048 50.292) (width 0.2) (layer "F.Cu") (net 10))
 (segment (start 130.905 49.245) (end 130.335 49.245) (width 0.2) (layer "F.Cu") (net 10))
 (segment (start 130.048 50.292) (end 128.27 52.07) (width 0.2) (layer "F.Cu") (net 10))
 (segment (start 129.902 46.812) (end 129.902 43.542) (width 0.2) (layer "F.Cu") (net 14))
 (segment (start 130.905 47.245) (end 130.335 47.245) (width 0.2) (layer "F.Cu") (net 14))
 (segment (start 129.902 43.542) (end 128.27 41.91) (width 0.2) (layer "F.Cu") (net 14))
 (segment (start 130.335 47.245) (end 129.902 46.812) (width 0.2) (layer "F.Cu") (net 14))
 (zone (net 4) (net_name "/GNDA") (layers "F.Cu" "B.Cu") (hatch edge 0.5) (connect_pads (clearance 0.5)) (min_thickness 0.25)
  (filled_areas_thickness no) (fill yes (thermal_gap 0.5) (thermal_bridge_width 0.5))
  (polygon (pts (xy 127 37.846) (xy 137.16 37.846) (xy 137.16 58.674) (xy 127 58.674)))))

